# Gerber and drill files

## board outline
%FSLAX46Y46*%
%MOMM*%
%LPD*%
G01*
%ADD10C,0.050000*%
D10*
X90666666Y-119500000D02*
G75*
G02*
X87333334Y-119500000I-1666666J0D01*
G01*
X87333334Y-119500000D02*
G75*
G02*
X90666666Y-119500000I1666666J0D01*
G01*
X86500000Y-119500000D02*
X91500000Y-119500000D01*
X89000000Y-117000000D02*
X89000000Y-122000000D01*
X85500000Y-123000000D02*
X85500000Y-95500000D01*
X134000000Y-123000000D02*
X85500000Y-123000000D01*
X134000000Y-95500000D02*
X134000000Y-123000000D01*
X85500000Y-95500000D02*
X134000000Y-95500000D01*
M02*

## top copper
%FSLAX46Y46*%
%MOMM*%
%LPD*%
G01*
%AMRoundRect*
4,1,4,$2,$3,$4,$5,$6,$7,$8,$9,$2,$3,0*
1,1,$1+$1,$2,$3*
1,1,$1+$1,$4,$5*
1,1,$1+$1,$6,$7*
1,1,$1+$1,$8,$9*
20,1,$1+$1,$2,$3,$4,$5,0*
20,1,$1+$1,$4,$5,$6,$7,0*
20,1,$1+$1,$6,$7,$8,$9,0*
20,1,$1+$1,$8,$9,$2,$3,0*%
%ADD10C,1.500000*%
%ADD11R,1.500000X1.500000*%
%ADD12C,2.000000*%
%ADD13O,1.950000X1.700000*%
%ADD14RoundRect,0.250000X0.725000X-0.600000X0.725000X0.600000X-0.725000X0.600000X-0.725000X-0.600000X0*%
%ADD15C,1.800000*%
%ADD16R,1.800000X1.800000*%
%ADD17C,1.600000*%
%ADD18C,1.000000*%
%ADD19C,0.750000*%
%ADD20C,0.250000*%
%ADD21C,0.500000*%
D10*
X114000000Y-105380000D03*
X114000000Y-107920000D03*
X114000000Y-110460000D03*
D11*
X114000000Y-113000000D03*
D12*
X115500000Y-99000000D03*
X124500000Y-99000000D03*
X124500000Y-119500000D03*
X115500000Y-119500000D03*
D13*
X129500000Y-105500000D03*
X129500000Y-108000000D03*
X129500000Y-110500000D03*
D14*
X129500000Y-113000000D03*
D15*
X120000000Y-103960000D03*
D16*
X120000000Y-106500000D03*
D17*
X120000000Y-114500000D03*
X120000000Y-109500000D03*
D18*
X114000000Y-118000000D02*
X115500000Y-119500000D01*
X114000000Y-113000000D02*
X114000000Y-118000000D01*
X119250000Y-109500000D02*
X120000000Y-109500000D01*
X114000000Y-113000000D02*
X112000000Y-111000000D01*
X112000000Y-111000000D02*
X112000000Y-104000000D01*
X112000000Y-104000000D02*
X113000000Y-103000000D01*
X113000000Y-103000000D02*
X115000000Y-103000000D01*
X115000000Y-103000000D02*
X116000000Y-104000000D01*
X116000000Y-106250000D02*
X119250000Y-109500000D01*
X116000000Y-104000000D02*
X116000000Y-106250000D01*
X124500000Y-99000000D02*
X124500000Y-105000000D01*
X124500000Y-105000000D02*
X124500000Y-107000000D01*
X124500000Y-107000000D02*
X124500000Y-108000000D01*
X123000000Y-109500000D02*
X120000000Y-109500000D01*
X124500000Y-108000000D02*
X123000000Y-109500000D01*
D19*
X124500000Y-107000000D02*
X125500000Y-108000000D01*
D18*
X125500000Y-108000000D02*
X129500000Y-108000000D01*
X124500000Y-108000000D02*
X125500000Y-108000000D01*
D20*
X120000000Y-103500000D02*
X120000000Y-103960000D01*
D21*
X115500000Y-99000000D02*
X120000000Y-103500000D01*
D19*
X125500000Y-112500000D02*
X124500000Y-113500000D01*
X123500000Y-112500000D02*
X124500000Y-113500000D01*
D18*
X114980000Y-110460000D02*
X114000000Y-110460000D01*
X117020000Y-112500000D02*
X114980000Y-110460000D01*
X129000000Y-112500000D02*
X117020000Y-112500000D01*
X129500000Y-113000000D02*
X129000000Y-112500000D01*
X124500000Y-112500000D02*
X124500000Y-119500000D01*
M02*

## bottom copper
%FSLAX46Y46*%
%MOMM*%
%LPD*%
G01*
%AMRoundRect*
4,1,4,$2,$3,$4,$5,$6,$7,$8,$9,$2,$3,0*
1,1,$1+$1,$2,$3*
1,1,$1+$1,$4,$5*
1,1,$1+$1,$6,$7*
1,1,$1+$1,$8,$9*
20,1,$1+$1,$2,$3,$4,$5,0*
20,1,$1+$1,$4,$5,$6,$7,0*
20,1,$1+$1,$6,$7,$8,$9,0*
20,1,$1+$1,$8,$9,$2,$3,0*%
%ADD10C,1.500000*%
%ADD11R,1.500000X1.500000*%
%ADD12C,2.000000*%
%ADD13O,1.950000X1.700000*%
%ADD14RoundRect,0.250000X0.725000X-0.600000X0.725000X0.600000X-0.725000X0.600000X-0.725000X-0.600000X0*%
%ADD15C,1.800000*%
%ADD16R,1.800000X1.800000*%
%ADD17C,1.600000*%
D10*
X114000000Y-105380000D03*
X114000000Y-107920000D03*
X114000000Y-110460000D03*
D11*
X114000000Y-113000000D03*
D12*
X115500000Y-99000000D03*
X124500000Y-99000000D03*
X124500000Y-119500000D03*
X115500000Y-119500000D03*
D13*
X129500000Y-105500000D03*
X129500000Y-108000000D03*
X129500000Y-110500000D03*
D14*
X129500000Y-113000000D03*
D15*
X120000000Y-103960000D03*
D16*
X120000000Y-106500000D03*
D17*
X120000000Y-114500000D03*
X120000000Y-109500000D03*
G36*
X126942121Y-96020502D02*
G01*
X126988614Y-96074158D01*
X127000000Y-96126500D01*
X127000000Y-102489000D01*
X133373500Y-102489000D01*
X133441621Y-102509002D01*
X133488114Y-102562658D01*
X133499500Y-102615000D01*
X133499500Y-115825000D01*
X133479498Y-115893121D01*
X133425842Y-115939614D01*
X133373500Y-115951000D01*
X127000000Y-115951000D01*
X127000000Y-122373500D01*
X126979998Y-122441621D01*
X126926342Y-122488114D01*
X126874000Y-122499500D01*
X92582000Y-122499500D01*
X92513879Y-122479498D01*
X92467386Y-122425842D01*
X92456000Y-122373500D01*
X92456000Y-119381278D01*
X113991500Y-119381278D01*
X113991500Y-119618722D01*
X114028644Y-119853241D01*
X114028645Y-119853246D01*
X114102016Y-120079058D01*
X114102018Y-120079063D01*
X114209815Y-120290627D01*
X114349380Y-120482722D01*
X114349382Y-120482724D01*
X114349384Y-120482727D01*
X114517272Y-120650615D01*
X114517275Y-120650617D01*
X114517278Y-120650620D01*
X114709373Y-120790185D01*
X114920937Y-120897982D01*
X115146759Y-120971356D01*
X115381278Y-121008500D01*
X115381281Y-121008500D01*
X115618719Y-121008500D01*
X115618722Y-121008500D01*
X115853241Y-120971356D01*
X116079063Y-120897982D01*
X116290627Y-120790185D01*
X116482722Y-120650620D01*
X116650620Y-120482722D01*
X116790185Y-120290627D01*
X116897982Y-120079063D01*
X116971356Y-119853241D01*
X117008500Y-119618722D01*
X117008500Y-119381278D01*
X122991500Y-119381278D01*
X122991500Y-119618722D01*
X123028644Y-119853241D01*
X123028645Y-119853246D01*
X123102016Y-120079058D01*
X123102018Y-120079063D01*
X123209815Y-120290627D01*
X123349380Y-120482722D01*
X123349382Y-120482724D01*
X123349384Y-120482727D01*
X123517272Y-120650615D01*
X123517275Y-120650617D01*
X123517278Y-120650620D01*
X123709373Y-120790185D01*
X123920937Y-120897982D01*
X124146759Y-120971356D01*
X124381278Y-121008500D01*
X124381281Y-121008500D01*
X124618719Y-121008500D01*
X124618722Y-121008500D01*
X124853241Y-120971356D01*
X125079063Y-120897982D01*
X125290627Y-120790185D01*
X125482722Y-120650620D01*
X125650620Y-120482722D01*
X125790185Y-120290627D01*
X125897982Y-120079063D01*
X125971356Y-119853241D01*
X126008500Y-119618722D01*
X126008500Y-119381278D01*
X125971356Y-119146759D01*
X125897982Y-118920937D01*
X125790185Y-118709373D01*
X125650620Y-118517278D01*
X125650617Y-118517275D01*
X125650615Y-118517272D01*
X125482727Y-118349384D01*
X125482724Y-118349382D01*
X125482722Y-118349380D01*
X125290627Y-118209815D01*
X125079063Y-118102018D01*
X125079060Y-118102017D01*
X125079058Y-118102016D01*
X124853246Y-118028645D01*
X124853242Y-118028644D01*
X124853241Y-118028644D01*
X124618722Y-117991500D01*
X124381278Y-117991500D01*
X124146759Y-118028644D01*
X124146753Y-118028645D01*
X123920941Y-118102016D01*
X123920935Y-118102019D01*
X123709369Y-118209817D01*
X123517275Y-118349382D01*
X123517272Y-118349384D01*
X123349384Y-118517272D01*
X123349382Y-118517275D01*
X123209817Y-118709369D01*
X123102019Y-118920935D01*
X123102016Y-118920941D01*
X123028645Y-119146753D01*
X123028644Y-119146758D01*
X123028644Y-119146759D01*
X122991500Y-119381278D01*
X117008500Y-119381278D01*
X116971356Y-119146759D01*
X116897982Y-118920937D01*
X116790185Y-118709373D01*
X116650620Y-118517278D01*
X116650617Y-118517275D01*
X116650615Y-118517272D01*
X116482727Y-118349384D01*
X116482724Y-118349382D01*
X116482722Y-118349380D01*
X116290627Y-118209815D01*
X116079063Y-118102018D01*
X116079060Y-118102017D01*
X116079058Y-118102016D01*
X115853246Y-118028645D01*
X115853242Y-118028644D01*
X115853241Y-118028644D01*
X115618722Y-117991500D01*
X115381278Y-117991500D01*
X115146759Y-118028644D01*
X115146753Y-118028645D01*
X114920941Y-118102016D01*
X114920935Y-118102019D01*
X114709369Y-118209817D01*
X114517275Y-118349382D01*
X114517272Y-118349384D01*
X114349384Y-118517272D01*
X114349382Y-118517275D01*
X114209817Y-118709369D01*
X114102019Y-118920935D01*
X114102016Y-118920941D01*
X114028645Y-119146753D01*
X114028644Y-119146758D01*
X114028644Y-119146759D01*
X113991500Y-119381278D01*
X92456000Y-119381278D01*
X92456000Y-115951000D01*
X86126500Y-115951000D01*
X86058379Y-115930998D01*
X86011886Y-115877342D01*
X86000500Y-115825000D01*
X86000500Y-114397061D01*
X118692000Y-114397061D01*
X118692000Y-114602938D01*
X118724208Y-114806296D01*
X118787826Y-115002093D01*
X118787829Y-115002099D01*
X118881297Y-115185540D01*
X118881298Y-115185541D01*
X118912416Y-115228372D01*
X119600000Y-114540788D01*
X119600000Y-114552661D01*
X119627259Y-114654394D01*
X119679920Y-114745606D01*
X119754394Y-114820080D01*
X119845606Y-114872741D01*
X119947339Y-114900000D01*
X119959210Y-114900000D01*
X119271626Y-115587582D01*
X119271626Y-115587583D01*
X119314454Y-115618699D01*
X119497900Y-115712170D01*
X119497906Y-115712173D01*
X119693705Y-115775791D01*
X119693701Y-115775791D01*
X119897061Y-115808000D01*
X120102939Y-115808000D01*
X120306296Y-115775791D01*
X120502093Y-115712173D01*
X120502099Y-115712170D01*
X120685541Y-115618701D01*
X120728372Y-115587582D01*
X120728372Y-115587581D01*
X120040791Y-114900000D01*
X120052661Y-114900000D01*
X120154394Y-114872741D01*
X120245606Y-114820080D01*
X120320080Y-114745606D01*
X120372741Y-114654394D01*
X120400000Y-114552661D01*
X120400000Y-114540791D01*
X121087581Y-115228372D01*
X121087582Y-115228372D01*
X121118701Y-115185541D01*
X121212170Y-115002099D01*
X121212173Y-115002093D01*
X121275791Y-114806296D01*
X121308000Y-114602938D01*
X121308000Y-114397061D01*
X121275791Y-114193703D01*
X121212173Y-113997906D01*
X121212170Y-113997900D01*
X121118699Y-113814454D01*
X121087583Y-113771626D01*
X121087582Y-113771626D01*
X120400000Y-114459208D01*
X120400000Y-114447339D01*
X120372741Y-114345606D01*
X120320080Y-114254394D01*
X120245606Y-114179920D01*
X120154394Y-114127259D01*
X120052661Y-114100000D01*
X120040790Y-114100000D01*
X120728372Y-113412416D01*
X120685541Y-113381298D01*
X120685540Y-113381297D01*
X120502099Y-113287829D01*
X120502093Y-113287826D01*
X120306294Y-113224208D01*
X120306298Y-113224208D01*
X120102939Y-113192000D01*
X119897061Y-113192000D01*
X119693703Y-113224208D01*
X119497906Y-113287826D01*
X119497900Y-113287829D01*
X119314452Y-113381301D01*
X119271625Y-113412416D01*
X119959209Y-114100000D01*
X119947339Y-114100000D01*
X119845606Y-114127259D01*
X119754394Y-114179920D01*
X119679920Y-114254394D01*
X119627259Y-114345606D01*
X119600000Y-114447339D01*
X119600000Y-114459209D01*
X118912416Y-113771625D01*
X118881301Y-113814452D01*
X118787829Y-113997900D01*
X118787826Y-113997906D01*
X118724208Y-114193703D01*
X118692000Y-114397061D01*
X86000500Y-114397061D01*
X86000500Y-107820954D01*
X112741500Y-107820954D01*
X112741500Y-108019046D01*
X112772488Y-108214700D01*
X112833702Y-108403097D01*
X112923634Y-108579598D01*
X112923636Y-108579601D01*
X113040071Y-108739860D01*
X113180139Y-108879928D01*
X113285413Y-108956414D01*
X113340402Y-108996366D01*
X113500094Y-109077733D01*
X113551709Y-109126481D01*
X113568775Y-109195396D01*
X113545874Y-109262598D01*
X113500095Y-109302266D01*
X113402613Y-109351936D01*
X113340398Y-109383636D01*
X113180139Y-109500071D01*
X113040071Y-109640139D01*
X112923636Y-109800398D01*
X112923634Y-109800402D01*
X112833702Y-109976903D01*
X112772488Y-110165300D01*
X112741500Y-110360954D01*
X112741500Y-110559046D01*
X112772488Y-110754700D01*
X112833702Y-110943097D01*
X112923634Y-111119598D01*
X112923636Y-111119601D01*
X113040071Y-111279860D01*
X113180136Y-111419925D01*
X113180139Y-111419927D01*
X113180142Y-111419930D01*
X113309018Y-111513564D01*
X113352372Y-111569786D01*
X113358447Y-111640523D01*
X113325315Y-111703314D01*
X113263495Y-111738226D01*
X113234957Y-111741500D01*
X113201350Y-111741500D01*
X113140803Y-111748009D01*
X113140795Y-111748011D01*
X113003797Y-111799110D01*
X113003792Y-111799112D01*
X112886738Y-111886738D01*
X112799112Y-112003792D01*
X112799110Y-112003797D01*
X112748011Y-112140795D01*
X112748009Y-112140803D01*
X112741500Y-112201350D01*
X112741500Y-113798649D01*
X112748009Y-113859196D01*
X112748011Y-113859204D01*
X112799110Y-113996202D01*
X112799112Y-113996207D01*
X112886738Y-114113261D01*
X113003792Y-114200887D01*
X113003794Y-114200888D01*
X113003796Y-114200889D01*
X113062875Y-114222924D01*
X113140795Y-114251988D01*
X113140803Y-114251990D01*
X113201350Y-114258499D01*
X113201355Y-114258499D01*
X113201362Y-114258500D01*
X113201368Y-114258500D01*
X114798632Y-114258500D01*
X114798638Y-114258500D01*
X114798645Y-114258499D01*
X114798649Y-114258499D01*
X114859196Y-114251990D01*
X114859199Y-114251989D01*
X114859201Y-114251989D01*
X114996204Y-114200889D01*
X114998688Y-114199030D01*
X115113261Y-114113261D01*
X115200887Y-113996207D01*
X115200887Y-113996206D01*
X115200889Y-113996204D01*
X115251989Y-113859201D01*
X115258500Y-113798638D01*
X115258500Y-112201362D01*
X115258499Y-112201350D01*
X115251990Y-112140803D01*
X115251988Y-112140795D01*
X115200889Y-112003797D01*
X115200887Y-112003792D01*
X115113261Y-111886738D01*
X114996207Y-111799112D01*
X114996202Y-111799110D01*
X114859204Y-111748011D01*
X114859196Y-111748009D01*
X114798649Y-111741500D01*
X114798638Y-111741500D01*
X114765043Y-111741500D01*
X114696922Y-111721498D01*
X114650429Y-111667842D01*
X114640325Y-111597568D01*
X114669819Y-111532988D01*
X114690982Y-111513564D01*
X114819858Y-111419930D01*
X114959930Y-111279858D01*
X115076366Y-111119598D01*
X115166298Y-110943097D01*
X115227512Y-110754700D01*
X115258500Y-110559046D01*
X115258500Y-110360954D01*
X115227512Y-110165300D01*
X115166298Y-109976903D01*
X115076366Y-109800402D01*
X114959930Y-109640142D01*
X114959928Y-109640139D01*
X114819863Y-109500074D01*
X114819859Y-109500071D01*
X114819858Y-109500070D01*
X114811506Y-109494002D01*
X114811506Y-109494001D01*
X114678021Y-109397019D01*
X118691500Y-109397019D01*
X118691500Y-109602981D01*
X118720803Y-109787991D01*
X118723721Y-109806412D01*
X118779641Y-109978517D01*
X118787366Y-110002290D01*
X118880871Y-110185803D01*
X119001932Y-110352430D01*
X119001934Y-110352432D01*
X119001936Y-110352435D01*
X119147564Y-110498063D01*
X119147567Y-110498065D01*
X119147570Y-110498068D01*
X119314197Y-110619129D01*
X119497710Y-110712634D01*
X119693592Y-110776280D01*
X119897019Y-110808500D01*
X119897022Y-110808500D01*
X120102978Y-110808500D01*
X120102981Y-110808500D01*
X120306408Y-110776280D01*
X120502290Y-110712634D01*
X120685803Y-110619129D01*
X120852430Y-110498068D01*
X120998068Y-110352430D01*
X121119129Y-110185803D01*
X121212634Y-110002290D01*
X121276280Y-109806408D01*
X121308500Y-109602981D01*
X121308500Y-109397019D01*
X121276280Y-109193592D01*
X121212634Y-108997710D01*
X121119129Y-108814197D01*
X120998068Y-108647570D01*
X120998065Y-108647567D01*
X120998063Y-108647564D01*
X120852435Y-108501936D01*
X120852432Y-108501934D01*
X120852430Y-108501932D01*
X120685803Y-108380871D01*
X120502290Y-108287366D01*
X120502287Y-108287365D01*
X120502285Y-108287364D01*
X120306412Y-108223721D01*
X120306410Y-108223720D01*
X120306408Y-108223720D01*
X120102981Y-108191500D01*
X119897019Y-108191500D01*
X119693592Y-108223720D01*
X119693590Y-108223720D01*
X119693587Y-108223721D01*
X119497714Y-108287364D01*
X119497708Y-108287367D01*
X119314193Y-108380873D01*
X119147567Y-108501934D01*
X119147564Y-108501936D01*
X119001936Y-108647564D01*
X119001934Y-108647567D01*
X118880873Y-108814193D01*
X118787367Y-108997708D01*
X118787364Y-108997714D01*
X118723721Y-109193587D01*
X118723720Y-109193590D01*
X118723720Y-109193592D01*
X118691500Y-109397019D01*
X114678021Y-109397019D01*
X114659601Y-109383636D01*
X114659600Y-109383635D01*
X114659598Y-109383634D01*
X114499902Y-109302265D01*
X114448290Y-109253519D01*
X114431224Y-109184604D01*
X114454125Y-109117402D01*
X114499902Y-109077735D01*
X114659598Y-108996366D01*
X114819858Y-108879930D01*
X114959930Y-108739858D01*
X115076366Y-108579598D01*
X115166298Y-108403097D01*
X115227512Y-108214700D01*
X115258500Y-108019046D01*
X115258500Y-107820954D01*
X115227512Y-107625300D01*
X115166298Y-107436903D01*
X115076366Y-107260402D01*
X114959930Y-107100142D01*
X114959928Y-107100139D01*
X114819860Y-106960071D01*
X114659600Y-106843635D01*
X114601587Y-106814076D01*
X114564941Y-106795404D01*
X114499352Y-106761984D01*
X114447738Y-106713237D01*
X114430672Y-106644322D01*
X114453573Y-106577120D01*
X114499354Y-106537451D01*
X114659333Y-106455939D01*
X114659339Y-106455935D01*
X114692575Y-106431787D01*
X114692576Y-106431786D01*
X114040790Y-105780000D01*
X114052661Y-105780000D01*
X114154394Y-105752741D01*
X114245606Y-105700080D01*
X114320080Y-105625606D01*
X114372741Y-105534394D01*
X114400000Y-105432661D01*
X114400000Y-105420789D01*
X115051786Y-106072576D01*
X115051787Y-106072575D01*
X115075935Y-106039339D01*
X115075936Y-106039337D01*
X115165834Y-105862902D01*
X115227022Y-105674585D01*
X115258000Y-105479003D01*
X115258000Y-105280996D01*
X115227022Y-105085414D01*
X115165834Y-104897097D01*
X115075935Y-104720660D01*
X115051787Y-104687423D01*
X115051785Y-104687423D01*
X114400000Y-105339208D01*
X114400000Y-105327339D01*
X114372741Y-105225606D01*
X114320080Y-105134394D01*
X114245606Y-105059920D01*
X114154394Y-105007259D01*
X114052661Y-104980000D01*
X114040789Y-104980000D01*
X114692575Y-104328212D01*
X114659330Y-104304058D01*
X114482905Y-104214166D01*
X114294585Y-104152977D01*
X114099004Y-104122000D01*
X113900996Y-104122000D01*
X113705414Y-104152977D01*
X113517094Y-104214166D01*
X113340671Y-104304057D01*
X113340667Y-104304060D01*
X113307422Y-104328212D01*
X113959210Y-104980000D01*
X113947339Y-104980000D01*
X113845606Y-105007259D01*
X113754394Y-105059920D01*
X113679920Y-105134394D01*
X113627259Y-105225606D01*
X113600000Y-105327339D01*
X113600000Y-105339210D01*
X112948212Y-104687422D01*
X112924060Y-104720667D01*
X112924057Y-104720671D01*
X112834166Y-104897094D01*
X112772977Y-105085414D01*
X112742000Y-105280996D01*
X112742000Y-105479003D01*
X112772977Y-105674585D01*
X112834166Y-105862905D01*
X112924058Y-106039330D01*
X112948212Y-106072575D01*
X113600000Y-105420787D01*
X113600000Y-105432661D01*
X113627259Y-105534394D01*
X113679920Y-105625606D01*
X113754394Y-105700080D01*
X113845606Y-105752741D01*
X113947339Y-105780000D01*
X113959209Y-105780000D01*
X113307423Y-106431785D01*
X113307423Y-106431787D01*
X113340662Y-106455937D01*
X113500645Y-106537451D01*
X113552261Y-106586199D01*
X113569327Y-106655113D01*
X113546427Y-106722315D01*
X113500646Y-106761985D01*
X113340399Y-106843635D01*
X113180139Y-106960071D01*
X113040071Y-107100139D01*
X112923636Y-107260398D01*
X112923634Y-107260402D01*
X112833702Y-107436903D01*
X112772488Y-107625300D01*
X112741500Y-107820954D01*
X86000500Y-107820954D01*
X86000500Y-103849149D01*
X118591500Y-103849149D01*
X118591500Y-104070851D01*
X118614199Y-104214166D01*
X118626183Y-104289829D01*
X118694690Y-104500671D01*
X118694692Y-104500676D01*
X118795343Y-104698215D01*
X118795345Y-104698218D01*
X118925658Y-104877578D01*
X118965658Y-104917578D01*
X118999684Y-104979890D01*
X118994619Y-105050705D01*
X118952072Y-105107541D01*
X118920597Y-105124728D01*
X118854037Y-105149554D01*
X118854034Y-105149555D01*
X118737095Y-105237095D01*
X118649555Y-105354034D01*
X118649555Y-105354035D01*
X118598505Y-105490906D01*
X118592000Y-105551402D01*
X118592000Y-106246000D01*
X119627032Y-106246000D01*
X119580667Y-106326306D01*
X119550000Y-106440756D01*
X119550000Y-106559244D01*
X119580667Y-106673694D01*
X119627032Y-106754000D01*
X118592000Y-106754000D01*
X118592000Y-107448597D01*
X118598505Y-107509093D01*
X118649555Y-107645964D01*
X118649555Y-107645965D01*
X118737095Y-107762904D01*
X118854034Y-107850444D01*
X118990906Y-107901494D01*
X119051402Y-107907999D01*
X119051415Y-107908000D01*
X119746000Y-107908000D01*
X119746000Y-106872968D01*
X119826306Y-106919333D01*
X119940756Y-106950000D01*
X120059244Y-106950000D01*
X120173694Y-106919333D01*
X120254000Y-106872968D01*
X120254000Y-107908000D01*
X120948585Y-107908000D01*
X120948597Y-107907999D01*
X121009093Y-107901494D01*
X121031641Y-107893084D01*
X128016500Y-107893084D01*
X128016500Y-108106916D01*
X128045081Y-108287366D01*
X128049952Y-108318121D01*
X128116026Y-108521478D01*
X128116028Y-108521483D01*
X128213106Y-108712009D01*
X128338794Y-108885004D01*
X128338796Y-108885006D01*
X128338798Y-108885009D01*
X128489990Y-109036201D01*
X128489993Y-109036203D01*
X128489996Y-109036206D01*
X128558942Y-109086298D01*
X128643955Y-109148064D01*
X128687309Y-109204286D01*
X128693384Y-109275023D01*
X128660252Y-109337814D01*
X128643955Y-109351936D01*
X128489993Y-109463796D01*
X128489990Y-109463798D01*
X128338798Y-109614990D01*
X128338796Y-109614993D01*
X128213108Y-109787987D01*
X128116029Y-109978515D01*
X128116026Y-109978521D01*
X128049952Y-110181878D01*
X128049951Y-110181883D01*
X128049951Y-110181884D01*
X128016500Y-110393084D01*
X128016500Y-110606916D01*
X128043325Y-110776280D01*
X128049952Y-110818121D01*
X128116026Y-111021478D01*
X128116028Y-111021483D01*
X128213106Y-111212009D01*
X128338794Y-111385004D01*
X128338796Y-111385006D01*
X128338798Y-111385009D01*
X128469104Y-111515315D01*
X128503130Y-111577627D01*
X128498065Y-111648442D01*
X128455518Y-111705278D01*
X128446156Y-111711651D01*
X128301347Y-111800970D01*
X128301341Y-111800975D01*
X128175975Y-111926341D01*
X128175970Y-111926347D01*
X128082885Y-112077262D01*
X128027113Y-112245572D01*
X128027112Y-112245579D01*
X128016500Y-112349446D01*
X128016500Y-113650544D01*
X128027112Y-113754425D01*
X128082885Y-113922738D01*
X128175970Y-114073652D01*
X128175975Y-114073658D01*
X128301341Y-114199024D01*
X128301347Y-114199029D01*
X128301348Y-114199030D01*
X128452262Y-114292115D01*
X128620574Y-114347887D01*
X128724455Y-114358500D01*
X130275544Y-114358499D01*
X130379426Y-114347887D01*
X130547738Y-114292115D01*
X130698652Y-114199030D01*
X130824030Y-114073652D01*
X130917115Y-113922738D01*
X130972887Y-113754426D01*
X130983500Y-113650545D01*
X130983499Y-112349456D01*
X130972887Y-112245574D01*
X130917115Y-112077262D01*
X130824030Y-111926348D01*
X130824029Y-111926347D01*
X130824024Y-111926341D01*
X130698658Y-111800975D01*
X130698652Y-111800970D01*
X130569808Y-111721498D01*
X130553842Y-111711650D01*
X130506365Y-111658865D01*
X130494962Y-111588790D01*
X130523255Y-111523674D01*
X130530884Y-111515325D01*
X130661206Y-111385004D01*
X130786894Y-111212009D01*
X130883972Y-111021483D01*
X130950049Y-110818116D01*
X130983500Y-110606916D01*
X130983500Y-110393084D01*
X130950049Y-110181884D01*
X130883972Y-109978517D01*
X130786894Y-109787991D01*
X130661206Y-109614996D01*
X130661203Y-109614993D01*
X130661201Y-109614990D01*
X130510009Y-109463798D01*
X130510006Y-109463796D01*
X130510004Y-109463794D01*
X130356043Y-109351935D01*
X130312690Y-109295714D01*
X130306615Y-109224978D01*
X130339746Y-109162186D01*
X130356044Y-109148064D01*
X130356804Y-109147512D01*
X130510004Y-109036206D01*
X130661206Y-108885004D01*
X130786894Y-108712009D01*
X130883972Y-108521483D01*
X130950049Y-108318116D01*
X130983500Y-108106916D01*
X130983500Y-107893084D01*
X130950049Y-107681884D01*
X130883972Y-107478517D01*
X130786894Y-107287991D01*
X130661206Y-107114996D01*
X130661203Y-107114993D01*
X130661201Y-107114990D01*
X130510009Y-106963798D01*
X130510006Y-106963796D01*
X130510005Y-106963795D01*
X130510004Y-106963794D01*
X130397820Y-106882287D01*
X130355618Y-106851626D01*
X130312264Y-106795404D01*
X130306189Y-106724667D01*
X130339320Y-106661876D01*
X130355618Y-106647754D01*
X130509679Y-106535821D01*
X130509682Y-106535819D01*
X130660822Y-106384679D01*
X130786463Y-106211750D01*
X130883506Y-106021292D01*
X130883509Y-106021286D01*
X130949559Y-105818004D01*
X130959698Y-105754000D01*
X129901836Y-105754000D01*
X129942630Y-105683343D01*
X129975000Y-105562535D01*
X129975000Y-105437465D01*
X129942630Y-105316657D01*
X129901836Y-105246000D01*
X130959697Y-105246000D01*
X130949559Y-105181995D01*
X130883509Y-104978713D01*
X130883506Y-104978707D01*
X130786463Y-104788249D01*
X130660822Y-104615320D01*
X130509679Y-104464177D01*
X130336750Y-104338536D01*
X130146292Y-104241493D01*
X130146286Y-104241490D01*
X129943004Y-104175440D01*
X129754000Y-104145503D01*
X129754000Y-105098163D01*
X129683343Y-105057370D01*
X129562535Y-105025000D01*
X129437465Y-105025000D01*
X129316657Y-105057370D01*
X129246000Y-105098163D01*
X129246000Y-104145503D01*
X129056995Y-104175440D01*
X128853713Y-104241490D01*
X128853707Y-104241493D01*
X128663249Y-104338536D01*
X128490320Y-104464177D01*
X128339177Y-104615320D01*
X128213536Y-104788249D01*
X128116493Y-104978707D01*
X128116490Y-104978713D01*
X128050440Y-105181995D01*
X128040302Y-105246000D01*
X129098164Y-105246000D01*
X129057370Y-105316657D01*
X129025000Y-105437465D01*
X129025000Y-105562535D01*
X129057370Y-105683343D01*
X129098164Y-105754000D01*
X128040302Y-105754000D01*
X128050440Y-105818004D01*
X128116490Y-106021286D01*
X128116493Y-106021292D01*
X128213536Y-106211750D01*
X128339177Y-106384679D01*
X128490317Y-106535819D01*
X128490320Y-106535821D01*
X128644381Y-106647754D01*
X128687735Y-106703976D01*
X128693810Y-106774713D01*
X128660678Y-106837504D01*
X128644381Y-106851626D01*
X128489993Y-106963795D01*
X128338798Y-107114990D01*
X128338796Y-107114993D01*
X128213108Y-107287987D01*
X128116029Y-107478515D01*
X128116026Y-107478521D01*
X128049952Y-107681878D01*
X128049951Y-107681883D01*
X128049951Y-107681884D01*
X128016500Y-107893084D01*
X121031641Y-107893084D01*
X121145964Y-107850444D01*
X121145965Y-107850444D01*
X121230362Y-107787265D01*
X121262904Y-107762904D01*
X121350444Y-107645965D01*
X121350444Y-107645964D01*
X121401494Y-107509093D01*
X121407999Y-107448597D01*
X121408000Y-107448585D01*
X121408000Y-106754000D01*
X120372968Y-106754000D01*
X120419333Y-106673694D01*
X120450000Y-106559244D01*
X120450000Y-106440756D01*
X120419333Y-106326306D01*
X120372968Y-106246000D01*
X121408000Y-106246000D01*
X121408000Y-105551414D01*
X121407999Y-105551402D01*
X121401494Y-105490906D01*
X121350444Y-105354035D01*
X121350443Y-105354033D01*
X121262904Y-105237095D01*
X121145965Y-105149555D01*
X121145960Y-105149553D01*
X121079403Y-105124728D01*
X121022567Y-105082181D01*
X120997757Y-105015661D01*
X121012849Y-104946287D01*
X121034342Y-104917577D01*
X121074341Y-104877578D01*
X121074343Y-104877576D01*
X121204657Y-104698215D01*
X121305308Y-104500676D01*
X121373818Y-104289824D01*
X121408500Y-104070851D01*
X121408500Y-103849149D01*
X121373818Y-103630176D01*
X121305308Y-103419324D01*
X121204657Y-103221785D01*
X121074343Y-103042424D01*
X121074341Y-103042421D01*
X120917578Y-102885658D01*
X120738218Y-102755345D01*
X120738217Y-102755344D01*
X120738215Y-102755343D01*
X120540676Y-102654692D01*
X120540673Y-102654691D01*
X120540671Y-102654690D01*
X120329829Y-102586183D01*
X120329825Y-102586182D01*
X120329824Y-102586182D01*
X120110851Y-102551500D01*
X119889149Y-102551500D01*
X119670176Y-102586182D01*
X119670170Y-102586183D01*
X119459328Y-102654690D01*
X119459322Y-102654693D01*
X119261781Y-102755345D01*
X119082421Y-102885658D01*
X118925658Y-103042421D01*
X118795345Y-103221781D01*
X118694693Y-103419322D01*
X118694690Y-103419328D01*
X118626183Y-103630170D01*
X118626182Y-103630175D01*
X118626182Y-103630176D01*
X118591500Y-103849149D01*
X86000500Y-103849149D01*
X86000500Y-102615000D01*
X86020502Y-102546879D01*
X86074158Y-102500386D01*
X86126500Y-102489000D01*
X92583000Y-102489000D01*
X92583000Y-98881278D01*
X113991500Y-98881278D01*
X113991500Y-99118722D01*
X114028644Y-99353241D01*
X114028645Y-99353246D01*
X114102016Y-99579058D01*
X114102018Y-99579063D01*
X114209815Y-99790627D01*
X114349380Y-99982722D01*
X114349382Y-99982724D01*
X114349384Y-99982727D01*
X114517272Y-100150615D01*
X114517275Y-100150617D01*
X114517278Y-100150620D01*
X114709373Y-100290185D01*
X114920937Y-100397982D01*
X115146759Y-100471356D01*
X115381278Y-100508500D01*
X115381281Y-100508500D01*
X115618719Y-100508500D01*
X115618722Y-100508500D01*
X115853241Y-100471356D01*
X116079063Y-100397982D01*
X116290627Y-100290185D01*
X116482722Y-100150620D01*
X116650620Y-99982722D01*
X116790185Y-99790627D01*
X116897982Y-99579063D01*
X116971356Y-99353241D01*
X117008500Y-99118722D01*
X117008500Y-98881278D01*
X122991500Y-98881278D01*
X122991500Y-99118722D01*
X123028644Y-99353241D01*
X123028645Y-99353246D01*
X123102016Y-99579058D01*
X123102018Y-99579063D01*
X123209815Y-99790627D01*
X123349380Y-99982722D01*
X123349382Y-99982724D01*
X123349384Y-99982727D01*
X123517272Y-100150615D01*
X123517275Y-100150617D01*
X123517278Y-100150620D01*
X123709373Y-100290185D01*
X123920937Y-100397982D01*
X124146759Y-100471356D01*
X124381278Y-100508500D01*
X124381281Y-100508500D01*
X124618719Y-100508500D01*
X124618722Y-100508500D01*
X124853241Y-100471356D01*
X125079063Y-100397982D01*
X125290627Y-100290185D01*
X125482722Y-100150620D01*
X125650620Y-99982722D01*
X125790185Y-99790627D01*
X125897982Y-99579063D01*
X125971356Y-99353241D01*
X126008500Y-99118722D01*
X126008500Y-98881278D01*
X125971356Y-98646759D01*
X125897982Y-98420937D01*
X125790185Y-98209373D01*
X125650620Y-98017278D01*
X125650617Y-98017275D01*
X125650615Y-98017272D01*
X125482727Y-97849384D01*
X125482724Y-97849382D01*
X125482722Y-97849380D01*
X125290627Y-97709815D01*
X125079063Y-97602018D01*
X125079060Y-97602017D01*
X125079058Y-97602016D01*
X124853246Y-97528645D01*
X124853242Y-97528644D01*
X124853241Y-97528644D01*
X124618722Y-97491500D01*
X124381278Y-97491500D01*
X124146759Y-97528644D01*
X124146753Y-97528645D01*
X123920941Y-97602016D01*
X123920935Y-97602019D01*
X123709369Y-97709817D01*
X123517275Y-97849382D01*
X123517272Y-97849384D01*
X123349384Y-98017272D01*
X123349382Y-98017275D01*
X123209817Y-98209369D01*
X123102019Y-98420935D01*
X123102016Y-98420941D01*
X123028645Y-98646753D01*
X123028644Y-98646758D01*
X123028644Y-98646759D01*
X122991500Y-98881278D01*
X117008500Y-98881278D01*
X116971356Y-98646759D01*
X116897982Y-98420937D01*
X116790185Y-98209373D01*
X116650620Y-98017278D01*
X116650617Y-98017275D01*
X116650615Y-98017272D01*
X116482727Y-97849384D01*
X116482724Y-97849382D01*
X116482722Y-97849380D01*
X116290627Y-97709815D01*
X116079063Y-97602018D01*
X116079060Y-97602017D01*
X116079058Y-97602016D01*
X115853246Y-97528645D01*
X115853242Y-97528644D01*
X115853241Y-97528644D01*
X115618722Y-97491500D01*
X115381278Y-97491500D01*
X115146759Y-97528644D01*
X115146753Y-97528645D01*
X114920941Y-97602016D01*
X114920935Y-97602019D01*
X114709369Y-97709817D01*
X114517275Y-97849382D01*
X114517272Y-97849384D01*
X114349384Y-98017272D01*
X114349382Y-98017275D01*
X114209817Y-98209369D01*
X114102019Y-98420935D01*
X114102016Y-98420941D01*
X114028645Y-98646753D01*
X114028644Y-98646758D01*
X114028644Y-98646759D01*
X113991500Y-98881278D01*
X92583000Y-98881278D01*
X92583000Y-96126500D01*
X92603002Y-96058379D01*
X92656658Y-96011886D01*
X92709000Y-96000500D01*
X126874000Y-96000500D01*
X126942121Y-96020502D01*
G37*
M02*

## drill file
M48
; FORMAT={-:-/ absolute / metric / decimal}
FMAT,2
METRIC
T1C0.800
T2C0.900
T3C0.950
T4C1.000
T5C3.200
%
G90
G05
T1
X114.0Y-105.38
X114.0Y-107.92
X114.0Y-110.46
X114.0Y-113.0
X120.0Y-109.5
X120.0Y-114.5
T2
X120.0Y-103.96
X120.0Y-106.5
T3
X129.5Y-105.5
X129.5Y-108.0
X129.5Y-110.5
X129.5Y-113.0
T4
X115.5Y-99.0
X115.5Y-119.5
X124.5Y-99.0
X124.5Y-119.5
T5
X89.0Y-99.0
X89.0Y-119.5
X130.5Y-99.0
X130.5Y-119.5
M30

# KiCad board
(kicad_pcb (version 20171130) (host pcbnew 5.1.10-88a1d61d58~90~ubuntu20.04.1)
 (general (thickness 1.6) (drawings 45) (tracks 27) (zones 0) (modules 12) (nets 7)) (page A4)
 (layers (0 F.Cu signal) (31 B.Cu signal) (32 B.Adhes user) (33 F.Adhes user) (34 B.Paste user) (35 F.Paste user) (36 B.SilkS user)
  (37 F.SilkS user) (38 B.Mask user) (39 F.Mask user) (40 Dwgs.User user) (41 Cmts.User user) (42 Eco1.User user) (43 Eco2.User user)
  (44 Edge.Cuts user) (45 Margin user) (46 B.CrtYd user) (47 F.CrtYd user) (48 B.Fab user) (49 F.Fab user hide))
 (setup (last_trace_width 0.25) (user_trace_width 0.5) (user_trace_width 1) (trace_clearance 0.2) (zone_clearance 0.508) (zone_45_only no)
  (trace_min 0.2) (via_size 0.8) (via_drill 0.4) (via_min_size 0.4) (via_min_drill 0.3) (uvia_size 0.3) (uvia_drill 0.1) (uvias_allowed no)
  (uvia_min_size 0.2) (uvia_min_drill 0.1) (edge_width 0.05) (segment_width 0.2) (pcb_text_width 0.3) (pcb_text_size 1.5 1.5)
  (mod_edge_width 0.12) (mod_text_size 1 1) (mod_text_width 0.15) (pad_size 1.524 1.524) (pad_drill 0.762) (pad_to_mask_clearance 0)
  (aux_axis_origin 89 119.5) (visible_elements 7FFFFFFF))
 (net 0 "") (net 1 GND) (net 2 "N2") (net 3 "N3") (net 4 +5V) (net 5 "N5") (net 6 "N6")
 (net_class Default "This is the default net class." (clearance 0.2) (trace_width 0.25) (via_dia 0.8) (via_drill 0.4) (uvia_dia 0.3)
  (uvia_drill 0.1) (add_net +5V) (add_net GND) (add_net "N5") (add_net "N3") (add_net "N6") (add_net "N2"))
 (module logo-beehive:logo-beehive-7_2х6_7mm (layer F.Cu) (at 98 119)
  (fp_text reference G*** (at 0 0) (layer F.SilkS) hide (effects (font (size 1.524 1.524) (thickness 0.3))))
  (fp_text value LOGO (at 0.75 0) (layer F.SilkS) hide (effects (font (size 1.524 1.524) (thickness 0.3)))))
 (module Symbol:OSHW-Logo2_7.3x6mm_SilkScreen (layer F.Cu) (at 106.5 119.5)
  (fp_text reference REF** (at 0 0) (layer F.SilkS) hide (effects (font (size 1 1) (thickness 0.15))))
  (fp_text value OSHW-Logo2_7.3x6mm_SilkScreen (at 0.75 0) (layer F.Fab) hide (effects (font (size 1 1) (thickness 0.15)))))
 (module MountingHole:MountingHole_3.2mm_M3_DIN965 (layer F.Cu) (at 89 119.5 180)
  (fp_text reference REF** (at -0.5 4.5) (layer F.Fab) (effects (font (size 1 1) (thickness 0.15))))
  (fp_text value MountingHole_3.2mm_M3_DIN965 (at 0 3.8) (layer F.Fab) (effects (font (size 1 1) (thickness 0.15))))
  (pad 1 np_thru_hole circle (at 0 0 180) (size 3.2 3.2) (drill 3.2) (layers *.Cu *.Mask)))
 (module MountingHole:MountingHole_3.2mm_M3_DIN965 (layer F.Cu) (at 89 99 90)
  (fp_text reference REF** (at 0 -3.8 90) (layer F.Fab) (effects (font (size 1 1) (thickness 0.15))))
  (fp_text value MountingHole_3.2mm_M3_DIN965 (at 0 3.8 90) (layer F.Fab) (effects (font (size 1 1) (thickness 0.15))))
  (pad 1 np_thru_hole circle (at 0 0 90) (size 3.2 3.2) (drill 3.2) (layers *.Cu *.Mask)))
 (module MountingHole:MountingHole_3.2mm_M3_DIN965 (layer F.Cu) (at 130.5 119.5)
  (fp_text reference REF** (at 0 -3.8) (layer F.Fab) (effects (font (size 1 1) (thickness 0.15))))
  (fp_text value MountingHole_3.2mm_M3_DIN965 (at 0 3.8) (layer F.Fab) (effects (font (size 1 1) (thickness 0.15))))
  (pad 1 np_thru_hole circle (at 0 0) (size 3.2 3.2) (drill 3.2) (layers *.Cu *.Mask)))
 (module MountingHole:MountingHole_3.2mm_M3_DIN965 (layer F.Cu) (at 130.5 99)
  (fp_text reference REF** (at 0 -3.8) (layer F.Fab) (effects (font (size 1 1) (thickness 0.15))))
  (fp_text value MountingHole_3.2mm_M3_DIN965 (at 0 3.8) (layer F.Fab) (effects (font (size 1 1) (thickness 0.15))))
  (pad 1 np_thru_hole circle (at 0 0) (size 3.2 3.2) (drill 3.2) (layers *.Cu *.Mask)))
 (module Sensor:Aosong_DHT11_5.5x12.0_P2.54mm (layer F.Cu) (at 114 113 180)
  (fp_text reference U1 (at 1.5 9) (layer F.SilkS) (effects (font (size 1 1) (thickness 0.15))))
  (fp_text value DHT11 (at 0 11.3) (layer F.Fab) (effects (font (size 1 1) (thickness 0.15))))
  (pad 4 thru_hole circle (at 0 7.62 180) (size 1.5 1.5) (drill 0.8) (layers *.Cu *.Mask) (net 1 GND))
  (pad 3 thru_hole circle (at 0 5.08 180) (size 1.5 1.5) (drill 0.8) (layers *.Cu *.Mask) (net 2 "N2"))
  (pad 2 thru_hole circle (at 0 2.54 180) (size 1.5 1.5) (drill 0.8) (layers *.Cu *.Mask) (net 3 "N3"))
  (pad 1 thru_hole rect (at 0 0 180) (size 1.5 1.5) (drill 0.8) (layers *.Cu *.Mask) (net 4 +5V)))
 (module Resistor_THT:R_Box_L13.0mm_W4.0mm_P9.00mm (layer F.Cu) (at 124.5 99 180)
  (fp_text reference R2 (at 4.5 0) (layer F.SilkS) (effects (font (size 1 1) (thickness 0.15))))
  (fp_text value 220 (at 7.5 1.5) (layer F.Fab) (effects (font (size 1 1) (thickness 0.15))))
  (pad 2 thru_hole circle (at 9 0 180) (size 2 2) (drill 1) (layers *.Cu *.Mask) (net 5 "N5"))
  (pad 1 thru_hole circle (at 0 0 180) (size 2 2) (drill 1) (layers *.Cu *.Mask) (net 4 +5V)))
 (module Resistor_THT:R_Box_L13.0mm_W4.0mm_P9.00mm (layer F.Cu) (at 115.5 119.5)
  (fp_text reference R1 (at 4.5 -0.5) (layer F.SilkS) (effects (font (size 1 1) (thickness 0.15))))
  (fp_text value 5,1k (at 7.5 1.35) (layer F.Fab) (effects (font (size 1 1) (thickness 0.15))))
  (pad 2 thru_hole circle (at 9 0) (size 2 2) (drill 1) (layers *.Cu *.Mask) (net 3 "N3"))
  (pad 1 thru_hole circle (at 0 0) (size 2 2) (drill 1) (layers *.Cu *.Mask) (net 4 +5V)))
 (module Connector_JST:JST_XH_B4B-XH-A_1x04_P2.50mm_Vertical (layer F.Cu) (at 129.5 113 90)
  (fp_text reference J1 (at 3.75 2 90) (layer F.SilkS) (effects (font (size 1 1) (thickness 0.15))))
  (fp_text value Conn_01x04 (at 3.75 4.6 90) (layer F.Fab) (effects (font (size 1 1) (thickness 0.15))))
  (pad 4 thru_hole oval (at 7.5 0 90) (size 1.7 1.95) (drill 0.95) (layers *.Cu *.Mask) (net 1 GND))
  (pad 3 thru_hole oval (at 5 0 90) (size 1.7 1.95) (drill 0.95) (layers *.Cu *.Mask) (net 4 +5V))
  (pad 2 thru_hole oval (at 2.5 0 90) (size 1.7 1.95) (drill 0.95) (layers *.Cu *.Mask) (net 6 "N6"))
  (pad 1 thru_hole roundrect (at 0 0 90) (size 1.7 1.95) (drill 0.95) (layers *.Cu *.Mask) (roundrect_rratio 0.1470588235294118)
   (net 3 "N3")))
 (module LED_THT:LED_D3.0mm (layer F.Cu) (at 120 106.5 90)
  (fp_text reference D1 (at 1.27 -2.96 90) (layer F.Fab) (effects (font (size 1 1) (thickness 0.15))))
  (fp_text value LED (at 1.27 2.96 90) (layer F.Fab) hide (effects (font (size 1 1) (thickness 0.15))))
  (pad 2 thru_hole circle (at 2.54 0 90) (size 1.8 1.8) (drill 0.9) (layers *.Cu *.Mask) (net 5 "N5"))
  (pad 1 thru_hole rect (at 0 0 90) (size 1.8 1.8) (drill 0.9) (layers *.Cu *.Mask) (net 1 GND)))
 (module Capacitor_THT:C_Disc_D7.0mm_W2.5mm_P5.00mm (layer F.Cu) (at 120 109.5 270)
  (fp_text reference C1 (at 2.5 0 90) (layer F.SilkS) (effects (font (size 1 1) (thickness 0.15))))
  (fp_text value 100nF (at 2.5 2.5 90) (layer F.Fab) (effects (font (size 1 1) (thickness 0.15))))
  (pad 2 thru_hole circle (at 5 0 270) (size 1.6 1.6) (drill 0.8) (layers *.Cu *.Mask) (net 1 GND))
  (pad 1 thru_hole circle (at 0 0 270) (size 1.6 1.6) (drill 0.8) (layers *.Cu *.Mask) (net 4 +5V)))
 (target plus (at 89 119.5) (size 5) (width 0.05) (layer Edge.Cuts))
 (gr_line (start 85.5 123) (end 85.5 95.5) (layer Edge.Cuts) (width 0.05))
 (gr_line (start 134 123) (end 85.5 123) (layer Edge.Cuts) (width 0.05))
 (gr_line (start 134 95.5) (end 134 123) (layer Edge.Cuts) (width 0.05))
 (gr_line (start 85.5 95.5) (end 134 95.5) (layer Edge.Cuts) (width 0.05))
 (segment (start 114 118) (end 115.5 119.5) (width 1) (layer F.Cu) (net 4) (status 20))
 (segment (start 114 113) (end 114 118) (width 1) (layer F.Cu) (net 4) (status 10))
 (segment (start 119.25 109.5) (end 120 109.5) (width 1) (layer F.Cu) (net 4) (status 30))
 (segment (start 114 113) (end 112 111) (width 1) (layer F.Cu) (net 4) (status 10))
 (segment (start 112 111) (end 112 104) (width 1) (layer F.Cu) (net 4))
 (segment (start 112 104) (end 113 103) (width 1) (layer F.Cu) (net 4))
 (segment (start 113 103) (end 115 103) (width 1) (layer F.Cu) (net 4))
 (segment (start 115 103) (end 116 104) (width 1) (layer F.Cu) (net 4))
 (segment (start 116 106.25) (end 119.25 109.5) (width 1) (layer F.Cu) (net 4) (status 20))
 (segment (start 116 104) (end 116 106.25) (width 1) (layer F.Cu) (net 4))
 (segment (start 124.5 99) (end 124.5 105) (width 1) (layer F.Cu) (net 4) (status 10))
 (segment (start 124.5 105) (end 124.5 107) (width 1) (layer F.Cu) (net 4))
 (segment (start 124.5 107) (end 124.5 108) (width 1) (layer F.Cu) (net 4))
 (segment (start 123 109.5) (end 120 109.5) (width 1) (layer F.Cu) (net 4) (status 20))
 (segment (start 124.5 108) (end 123 109.5) (width 1) (layer F.Cu) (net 4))
 (segment (start 124.5 107) (end 125.5 108) (width 0.75) (layer F.Cu) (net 4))
 (segment (start 125.5 108) (end 129.5 108) (width 1) (layer F.Cu) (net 4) (status 20))
 (segment (start 124.5 108) (end 125.5 108) (width 1) (layer F.Cu) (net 4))
 (segment (start 120 103.5) (end 120 103.96) (width 0.25) (layer F.Cu) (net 5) (status 30))
 (segment (start 115.5 99) (end 120 103.5) (width 0.5) (layer F.Cu) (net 5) (status 30))
 (segment (start 125.5 112.5) (end 124.5 113.5) (width 0.75) (layer F.Cu) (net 3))
 (segment (start 123.5 112.5) (end 124.5 113.5) (width 0.75) (layer F.Cu) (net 3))
 (segment (start 114.98 110.46) (end 114 110.46) (width 1) (layer F.Cu) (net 3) (status 20))
 (segment (start 117.02 112.5) (end 114.98 110.46) (width 1) (layer F.Cu) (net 3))
 (segment (start 129 112.5) (end 117.02 112.5) (width 1) (layer F.Cu) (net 3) (status 10))
 (segment (start 129.5 113) (end 129 112.5) (width 1) (layer F.Cu) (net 3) (status 30))
 (segment (start 124.5 112.5) (end 124.5 119.5) (width 1) (layer F.Cu) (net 3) (status 20))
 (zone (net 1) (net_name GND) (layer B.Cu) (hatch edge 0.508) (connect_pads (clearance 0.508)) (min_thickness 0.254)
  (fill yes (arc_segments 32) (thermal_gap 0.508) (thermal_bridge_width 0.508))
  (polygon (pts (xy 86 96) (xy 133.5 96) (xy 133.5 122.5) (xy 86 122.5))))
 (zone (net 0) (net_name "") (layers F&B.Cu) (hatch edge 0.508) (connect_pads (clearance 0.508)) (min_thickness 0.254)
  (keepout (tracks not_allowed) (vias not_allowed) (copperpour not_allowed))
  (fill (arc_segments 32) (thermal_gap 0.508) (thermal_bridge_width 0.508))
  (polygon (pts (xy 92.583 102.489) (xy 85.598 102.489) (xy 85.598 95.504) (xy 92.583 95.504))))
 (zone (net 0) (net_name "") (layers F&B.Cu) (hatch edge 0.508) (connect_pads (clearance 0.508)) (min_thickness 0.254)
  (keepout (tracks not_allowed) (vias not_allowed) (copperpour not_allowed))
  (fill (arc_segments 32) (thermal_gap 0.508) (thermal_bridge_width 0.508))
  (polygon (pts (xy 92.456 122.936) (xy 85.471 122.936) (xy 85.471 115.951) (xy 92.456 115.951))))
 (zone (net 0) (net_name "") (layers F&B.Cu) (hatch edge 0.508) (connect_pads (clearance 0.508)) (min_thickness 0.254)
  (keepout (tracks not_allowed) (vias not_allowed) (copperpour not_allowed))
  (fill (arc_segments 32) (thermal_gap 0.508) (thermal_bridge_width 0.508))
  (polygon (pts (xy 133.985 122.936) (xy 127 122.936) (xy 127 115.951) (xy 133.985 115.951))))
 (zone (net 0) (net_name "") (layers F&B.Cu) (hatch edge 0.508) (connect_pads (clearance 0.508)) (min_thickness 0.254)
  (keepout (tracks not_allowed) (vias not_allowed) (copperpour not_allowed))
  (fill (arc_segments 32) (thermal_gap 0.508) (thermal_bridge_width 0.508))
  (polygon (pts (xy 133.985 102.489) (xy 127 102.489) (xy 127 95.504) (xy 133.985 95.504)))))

